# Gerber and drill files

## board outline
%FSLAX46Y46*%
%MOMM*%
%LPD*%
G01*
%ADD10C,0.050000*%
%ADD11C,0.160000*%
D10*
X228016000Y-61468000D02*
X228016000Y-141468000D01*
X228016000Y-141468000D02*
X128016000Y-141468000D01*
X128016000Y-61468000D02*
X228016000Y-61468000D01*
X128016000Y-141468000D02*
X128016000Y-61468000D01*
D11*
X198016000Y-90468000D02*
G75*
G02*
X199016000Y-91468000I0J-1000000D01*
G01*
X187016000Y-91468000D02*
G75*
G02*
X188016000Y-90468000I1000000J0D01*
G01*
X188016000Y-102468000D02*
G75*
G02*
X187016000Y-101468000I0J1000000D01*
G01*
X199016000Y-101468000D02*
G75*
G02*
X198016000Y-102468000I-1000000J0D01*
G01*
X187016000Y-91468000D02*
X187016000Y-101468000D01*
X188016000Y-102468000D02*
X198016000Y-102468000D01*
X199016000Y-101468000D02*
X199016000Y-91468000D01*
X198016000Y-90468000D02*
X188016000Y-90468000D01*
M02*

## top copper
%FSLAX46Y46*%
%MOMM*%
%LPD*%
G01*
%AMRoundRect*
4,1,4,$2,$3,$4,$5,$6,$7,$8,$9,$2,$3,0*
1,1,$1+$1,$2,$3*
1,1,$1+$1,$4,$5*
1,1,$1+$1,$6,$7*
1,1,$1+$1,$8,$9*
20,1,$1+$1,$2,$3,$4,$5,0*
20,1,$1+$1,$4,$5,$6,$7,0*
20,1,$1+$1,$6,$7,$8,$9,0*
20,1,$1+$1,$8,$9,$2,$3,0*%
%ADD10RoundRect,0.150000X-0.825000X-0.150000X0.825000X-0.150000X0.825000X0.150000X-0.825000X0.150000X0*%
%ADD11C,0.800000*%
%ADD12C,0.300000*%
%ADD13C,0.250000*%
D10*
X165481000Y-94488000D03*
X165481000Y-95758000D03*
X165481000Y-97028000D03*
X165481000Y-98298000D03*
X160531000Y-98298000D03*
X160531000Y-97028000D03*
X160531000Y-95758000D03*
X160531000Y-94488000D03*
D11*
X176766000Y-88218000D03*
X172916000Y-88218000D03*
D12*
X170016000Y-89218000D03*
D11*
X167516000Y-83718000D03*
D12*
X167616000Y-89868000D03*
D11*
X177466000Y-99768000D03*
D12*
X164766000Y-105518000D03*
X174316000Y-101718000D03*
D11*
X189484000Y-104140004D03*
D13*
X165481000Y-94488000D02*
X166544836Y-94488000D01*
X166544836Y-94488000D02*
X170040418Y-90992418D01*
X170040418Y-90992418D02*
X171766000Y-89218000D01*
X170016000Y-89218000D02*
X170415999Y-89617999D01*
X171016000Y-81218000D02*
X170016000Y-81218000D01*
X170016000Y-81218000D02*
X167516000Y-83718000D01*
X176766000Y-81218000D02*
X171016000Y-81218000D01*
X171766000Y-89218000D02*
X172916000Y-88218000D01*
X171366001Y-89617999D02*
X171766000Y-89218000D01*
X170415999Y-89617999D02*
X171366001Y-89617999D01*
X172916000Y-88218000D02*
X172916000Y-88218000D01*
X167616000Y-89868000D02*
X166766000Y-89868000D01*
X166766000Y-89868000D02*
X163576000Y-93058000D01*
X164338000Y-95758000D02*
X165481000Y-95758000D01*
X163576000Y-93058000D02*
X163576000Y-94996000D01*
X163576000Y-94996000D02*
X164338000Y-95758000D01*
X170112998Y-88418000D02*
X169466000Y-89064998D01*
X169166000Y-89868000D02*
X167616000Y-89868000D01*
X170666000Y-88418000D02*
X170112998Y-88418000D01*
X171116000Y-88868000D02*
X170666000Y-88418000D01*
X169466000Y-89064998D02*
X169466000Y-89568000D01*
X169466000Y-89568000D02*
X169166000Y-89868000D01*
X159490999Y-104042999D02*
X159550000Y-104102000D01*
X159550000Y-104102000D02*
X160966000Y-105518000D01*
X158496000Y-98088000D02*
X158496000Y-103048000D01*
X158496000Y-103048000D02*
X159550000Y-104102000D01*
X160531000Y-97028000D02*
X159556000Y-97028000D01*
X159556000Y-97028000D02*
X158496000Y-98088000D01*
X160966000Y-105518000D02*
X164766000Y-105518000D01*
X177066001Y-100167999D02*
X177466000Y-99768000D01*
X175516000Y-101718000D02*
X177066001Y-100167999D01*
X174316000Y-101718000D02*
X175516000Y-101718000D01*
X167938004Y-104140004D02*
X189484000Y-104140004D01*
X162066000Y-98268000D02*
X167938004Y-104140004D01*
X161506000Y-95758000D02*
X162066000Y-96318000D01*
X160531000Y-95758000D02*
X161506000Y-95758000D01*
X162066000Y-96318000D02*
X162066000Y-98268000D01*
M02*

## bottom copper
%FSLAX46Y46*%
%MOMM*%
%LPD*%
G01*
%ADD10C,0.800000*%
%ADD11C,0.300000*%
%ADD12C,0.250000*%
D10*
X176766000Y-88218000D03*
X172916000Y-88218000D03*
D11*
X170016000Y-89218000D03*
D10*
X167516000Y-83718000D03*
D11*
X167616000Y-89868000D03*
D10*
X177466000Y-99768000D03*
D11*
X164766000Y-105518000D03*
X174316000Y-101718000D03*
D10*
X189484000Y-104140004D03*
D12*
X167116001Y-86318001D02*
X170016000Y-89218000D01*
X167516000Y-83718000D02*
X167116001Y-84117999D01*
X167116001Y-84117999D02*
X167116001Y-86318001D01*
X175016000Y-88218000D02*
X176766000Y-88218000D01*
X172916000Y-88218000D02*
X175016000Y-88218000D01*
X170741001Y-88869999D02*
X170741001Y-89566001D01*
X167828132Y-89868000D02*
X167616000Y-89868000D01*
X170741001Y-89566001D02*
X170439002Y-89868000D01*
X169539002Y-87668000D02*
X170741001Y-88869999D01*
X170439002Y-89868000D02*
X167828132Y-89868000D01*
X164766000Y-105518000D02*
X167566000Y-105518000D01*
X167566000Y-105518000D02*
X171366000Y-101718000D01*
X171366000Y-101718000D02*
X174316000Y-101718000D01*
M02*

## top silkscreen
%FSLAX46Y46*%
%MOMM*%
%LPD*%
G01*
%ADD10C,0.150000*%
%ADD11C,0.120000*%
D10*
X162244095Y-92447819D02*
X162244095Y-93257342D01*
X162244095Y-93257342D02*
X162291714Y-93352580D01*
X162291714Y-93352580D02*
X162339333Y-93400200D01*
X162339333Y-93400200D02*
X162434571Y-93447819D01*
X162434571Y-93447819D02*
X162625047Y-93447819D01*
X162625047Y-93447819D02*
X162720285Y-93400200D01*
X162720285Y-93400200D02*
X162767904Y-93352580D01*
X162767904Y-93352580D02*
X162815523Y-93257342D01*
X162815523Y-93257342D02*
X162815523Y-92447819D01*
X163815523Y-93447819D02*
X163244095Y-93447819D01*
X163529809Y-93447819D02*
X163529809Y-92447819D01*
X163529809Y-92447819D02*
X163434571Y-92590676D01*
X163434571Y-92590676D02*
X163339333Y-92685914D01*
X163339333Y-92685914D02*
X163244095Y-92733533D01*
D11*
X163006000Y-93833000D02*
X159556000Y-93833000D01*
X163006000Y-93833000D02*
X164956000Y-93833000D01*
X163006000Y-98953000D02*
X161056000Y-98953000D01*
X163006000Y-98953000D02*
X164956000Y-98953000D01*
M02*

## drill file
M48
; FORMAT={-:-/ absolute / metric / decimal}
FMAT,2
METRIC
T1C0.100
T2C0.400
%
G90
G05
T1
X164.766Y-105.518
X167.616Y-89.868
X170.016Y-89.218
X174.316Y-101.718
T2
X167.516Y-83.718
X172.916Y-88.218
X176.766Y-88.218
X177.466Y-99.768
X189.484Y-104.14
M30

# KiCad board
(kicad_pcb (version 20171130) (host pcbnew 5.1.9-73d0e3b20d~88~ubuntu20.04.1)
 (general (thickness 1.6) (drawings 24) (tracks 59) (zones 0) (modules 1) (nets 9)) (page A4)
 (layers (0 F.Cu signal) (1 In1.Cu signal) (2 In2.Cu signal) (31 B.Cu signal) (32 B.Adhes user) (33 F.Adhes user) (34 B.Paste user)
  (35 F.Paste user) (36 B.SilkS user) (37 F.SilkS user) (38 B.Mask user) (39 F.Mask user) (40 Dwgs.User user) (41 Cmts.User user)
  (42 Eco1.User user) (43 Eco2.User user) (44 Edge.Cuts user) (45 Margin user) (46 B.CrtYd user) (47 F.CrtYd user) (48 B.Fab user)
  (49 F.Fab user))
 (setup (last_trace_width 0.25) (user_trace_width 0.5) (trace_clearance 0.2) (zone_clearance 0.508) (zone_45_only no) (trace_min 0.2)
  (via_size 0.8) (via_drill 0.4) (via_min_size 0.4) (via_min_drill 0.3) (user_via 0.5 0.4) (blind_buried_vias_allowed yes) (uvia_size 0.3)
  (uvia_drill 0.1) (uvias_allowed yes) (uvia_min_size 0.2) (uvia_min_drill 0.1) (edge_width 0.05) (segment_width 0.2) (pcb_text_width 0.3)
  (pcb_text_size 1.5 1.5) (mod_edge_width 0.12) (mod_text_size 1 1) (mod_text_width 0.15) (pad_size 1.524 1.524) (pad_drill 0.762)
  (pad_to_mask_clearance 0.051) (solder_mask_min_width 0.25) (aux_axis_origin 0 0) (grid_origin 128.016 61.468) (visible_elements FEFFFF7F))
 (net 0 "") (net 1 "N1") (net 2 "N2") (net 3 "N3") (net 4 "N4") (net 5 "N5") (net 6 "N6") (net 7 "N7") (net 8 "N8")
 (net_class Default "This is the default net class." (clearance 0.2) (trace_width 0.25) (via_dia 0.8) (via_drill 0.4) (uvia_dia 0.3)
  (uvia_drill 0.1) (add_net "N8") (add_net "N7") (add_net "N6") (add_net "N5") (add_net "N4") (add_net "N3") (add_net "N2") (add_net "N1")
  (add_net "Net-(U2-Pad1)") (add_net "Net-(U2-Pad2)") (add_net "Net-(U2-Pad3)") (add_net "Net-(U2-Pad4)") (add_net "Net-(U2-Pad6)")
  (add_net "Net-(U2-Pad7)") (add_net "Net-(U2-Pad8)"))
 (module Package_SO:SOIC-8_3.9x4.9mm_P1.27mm (layer F.Cu) (at 163.006 96.393)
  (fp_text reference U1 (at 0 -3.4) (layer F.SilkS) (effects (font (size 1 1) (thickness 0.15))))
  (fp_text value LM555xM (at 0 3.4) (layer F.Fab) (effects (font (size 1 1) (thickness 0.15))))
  (fp_line (start 0 -2.56) (end -3.45 -2.56) (layer F.SilkS) (width 0.12))
  (fp_line (start 0 -2.56) (end 1.95 -2.56) (layer F.SilkS) (width 0.12))
  (fp_line (start 0 2.56) (end -1.95 2.56) (layer F.SilkS) (width 0.12))
  (fp_line (start 0 2.56) (end 1.95 2.56) (layer F.SilkS) (width 0.12))
  (pad 8 smd roundrect (at 2.475 -1.905) (size 1.95 0.6) (layers F.Cu F.Paste F.Mask) (roundrect_rratio 0.25) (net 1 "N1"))
  (pad 7 smd roundrect (at 2.475 -0.635) (size 1.95 0.6) (layers F.Cu F.Paste F.Mask) (roundrect_rratio 0.25) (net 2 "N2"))
  (pad 6 smd roundrect (at 2.475 0.635) (size 1.95 0.6) (layers F.Cu F.Paste F.Mask) (roundrect_rratio 0.25) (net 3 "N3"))
  (pad 5 smd roundrect (at 2.475 1.905) (size 1.95 0.6) (layers F.Cu F.Paste F.Mask) (roundrect_rratio 0.25) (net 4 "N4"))
  (pad 4 smd roundrect (at -2.475 1.905) (size 1.95 0.6) (layers F.Cu F.Paste F.Mask) (roundrect_rratio 0.25) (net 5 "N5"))
  (pad 3 smd roundrect (at -2.475 0.635) (size 1.95 0.6) (layers F.Cu F.Paste F.Mask) (roundrect_rratio 0.25) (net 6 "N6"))
  (pad 2 smd roundrect (at -2.475 -0.635) (size 1.95 0.6) (layers F.Cu F.Paste F.Mask) (roundrect_rratio 0.25) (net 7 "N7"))
  (pad 1 smd roundrect (at -2.475 -1.905) (size 1.95 0.6) (layers F.Cu F.Paste F.Mask) (roundrect_rratio 0.25) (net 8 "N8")))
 (gr_line (start 228.016 61.468) (end 228.016 141.468) (layer Edge.Cuts) (width 0.05))
 (gr_line (start 228.016 141.468) (end 128.016 141.468) (layer Edge.Cuts) (width 0.05))
 (gr_line (start 128.016 61.468) (end 228.016 61.468) (layer Edge.Cuts) (width 0.05))
 (gr_line (start 128.016 141.468) (end 128.016 61.468) (layer Edge.Cuts) (width 0.05))
 (gr_arc (start 198.016 91.468) (end 199.016 91.468) (angle -90) (layer Edge.Cuts) (width 0.16))
 (gr_arc (start 188.016 91.468) (end 188.016 90.468) (angle -90) (layer Edge.Cuts) (width 0.16))
 (gr_arc (start 188.016 101.468) (end 187.016 101.468) (angle -90) (layer Edge.Cuts) (width 0.16))
 (gr_arc (start 198.016 101.468) (end 198.016 102.468) (angle -90) (layer Edge.Cuts) (width 0.16))
 (gr_line (start 187.016 91.468) (end 187.016 101.468) (angle 90) (layer Edge.Cuts) (width 0.16))
 (gr_line (start 188.016 102.468) (end 198.016 102.468) (angle 90) (layer Edge.Cuts) (width 0.16))
 (gr_line (start 199.016 101.468) (end 199.016 91.468) (angle 90) (layer Edge.Cuts) (width 0.16))
 (gr_line (start 198.016 90.468) (end 188.016 90.468) (angle 90) (layer Edge.Cuts) (width 0.16))
 (via (at 176.766 88.218) (size 0.8) (drill 0.4) (layers F.Cu B.Cu) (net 1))
 (segment (start 165.481 94.488) (end 166.544836 94.488) (width 0.25) (layer F.Cu) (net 1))
 (segment (start 166.544836 94.488) (end 170.040418 90.992418) (width 0.25) (layer F.Cu) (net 1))
 (segment (start 170.040418 90.992418) (end 171.766 89.218) (width 0.25) (layer F.Cu) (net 1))
 (segment (start 170.016 89.218) (end 170.415999 89.617999) (width 0.25) (layer F.Cu) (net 1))
 (segment (start 167.116001 86.318001) (end 170.016 89.218) (width 0.25) (layer B.Cu) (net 1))
 (segment (start 167.516 83.718) (end 167.116001 84.117999) (width 0.25) (layer B.Cu) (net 1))
 (segment (start 167.116001 84.117999) (end 167.116001 86.318001) (width 0.25) (layer B.Cu) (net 1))
 (segment (start 171.016 81.218) (end 170.016 81.218) (width 0.25) (layer F.Cu) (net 1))
 (segment (start 170.016 81.218) (end 167.516 83.718) (width 0.25) (layer F.Cu) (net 1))
 (segment (start 176.766 81.218) (end 171.016 81.218) (width 0.25) (layer F.Cu) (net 1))
 (via (at 172.916 88.218) (size 0.8) (drill 0.4) (layers F.Cu B.Cu) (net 1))
 (segment (start 171.766 89.218) (end 172.916 88.218) (width 0.25) (layer F.Cu) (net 1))
 (segment (start 171.366001 89.617999) (end 171.766 89.218) (width 0.25) (layer F.Cu) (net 1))
 (segment (start 170.415999 89.617999) (end 171.366001 89.617999) (width 0.25) (layer F.Cu) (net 1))
 (via (at 170.016 89.218) (size 0.3) (drill 0.1) (layers F.Cu B.Cu) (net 1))
 (via (at 167.516 83.718) (size 0.8) (drill 0.4) (layers F.Cu B.Cu) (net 1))
 (segment (start 175.016 88.218) (end 176.766 88.218) (width 0.25) (layer B.Cu) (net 1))
 (segment (start 172.916 88.218) (end 172.916 88.218) (width 0.25) (layer F.Cu) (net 1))
 (segment (start 172.916 88.218) (end 175.016 88.218) (width 0.25) (layer B.Cu) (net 1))
 (segment (start 167.616 89.868) (end 166.766 89.868) (width 0.25) (layer F.Cu) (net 2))
 (segment (start 166.766 89.868) (end 163.576 93.058) (width 0.25) (layer F.Cu) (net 2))
 (segment (start 164.338 95.758) (end 165.481 95.758) (width 0.25) (layer F.Cu) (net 2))
 (segment (start 163.576 93.058) (end 163.576 94.996) (width 0.25) (layer F.Cu) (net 2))
 (segment (start 163.576 94.996) (end 164.338 95.758) (width 0.25) (layer F.Cu) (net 2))
 (segment (start 170.112998 88.418) (end 169.466 89.064998) (width 0.25) (layer F.Cu) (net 2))
 (segment (start 169.166 89.868) (end 167.616 89.868) (width 0.25) (layer F.Cu) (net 2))
 (segment (start 170.666 88.418) (end 170.112998 88.418) (width 0.25) (layer F.Cu) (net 2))
 (segment (start 171.116 88.868) (end 170.666 88.418) (width 0.25) (layer F.Cu) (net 2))
 (segment (start 169.466 89.064998) (end 169.466 89.568) (width 0.25) (layer F.Cu) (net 2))
 (segment (start 170.741001 88.869999) (end 170.741001 89.566001) (width 0.25) (layer B.Cu) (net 2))
 (via (at 167.616 89.868) (size 0.3) (drill 0.1) (layers F.Cu B.Cu) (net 2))
 (segment (start 167.828132 89.868) (end 167.616 89.868) (width 0.25) (layer B.Cu) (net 2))
 (segment (start 170.741001 89.566001) (end 170.439002 89.868) (width 0.25) (layer B.Cu) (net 2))
 (segment (start 169.539002 87.668) (end 170.741001 88.869999) (width 0.25) (layer B.Cu) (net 2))
 (segment (start 170.439002 89.868) (end 167.828132 89.868) (width 0.25) (layer B.Cu) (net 2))
 (segment (start 169.466 89.568) (end 169.166 89.868) (width 0.25) (layer F.Cu) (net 2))
 (via (at 177.466 99.768) (size 0.8) (drill 0.4) (layers F.Cu B.Cu) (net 6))
 (segment (start 159.490999 104.042999) (end 159.55 104.102) (width 0.25) (layer F.Cu) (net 6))
 (segment (start 159.55 104.102) (end 160.966 105.518) (width 0.25) (layer F.Cu) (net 6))
 (segment (start 158.496 98.088) (end 158.496 103.048) (width 0.25) (layer F.Cu) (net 6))
 (segment (start 158.496 103.048) (end 159.55 104.102) (width 0.25) (layer F.Cu) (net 6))
 (segment (start 160.531 97.028) (end 159.556 97.028) (width 0.25) (layer F.Cu) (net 6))
 (segment (start 159.556 97.028) (end 158.496 98.088) (width 0.25) (layer F.Cu) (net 6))
 (segment (start 164.766 105.518) (end 167.566 105.518) (width 0.25) (layer B.Cu) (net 6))
 (segment (start 167.566 105.518) (end 171.366 101.718) (width 0.25) (layer B.Cu) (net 6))
 (segment (start 171.366 101.718) (end 174.316 101.718) (width 0.25) (layer B.Cu) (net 6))
 (via (at 164.766 105.518) (size 0.3) (drill 0.1) (layers F.Cu B.Cu) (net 6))
 (segment (start 160.966 105.518) (end 164.766 105.518) (width 0.25) (layer F.Cu) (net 6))
 (via (at 174.316 101.718) (size 0.3) (drill 0.1) (layers F.Cu B.Cu) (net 6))
 (segment (start 177.066001 100.167999) (end 177.466 99.768) (width 0.25) (layer F.Cu) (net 6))
 (segment (start 175.516 101.718) (end 177.066001 100.167999) (width 0.25) (layer F.Cu) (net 6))
 (segment (start 174.316 101.718) (end 175.516 101.718) (width 0.25) (layer F.Cu) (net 6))
 (via (at 189.484 104.140004) (size 0.8) (drill 0.4) (layers F.Cu B.Cu) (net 7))
 (segment (start 167.938004 104.140004) (end 189.484 104.140004) (width 0.25) (layer F.Cu) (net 7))
 (segment (start 162.066 98.268) (end 167.938004 104.140004) (width 0.25) (layer F.Cu) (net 7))
 (segment (start 161.506 95.758) (end 162.066 96.318) (width 0.25) (layer F.Cu) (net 7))
 (segment (start 160.531 95.758) (end 161.506 95.758) (width 0.25) (layer F.Cu) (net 7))
 (segment (start 162.066 96.318) (end 162.066 98.268) (width 0.25) (layer F.Cu) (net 7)))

